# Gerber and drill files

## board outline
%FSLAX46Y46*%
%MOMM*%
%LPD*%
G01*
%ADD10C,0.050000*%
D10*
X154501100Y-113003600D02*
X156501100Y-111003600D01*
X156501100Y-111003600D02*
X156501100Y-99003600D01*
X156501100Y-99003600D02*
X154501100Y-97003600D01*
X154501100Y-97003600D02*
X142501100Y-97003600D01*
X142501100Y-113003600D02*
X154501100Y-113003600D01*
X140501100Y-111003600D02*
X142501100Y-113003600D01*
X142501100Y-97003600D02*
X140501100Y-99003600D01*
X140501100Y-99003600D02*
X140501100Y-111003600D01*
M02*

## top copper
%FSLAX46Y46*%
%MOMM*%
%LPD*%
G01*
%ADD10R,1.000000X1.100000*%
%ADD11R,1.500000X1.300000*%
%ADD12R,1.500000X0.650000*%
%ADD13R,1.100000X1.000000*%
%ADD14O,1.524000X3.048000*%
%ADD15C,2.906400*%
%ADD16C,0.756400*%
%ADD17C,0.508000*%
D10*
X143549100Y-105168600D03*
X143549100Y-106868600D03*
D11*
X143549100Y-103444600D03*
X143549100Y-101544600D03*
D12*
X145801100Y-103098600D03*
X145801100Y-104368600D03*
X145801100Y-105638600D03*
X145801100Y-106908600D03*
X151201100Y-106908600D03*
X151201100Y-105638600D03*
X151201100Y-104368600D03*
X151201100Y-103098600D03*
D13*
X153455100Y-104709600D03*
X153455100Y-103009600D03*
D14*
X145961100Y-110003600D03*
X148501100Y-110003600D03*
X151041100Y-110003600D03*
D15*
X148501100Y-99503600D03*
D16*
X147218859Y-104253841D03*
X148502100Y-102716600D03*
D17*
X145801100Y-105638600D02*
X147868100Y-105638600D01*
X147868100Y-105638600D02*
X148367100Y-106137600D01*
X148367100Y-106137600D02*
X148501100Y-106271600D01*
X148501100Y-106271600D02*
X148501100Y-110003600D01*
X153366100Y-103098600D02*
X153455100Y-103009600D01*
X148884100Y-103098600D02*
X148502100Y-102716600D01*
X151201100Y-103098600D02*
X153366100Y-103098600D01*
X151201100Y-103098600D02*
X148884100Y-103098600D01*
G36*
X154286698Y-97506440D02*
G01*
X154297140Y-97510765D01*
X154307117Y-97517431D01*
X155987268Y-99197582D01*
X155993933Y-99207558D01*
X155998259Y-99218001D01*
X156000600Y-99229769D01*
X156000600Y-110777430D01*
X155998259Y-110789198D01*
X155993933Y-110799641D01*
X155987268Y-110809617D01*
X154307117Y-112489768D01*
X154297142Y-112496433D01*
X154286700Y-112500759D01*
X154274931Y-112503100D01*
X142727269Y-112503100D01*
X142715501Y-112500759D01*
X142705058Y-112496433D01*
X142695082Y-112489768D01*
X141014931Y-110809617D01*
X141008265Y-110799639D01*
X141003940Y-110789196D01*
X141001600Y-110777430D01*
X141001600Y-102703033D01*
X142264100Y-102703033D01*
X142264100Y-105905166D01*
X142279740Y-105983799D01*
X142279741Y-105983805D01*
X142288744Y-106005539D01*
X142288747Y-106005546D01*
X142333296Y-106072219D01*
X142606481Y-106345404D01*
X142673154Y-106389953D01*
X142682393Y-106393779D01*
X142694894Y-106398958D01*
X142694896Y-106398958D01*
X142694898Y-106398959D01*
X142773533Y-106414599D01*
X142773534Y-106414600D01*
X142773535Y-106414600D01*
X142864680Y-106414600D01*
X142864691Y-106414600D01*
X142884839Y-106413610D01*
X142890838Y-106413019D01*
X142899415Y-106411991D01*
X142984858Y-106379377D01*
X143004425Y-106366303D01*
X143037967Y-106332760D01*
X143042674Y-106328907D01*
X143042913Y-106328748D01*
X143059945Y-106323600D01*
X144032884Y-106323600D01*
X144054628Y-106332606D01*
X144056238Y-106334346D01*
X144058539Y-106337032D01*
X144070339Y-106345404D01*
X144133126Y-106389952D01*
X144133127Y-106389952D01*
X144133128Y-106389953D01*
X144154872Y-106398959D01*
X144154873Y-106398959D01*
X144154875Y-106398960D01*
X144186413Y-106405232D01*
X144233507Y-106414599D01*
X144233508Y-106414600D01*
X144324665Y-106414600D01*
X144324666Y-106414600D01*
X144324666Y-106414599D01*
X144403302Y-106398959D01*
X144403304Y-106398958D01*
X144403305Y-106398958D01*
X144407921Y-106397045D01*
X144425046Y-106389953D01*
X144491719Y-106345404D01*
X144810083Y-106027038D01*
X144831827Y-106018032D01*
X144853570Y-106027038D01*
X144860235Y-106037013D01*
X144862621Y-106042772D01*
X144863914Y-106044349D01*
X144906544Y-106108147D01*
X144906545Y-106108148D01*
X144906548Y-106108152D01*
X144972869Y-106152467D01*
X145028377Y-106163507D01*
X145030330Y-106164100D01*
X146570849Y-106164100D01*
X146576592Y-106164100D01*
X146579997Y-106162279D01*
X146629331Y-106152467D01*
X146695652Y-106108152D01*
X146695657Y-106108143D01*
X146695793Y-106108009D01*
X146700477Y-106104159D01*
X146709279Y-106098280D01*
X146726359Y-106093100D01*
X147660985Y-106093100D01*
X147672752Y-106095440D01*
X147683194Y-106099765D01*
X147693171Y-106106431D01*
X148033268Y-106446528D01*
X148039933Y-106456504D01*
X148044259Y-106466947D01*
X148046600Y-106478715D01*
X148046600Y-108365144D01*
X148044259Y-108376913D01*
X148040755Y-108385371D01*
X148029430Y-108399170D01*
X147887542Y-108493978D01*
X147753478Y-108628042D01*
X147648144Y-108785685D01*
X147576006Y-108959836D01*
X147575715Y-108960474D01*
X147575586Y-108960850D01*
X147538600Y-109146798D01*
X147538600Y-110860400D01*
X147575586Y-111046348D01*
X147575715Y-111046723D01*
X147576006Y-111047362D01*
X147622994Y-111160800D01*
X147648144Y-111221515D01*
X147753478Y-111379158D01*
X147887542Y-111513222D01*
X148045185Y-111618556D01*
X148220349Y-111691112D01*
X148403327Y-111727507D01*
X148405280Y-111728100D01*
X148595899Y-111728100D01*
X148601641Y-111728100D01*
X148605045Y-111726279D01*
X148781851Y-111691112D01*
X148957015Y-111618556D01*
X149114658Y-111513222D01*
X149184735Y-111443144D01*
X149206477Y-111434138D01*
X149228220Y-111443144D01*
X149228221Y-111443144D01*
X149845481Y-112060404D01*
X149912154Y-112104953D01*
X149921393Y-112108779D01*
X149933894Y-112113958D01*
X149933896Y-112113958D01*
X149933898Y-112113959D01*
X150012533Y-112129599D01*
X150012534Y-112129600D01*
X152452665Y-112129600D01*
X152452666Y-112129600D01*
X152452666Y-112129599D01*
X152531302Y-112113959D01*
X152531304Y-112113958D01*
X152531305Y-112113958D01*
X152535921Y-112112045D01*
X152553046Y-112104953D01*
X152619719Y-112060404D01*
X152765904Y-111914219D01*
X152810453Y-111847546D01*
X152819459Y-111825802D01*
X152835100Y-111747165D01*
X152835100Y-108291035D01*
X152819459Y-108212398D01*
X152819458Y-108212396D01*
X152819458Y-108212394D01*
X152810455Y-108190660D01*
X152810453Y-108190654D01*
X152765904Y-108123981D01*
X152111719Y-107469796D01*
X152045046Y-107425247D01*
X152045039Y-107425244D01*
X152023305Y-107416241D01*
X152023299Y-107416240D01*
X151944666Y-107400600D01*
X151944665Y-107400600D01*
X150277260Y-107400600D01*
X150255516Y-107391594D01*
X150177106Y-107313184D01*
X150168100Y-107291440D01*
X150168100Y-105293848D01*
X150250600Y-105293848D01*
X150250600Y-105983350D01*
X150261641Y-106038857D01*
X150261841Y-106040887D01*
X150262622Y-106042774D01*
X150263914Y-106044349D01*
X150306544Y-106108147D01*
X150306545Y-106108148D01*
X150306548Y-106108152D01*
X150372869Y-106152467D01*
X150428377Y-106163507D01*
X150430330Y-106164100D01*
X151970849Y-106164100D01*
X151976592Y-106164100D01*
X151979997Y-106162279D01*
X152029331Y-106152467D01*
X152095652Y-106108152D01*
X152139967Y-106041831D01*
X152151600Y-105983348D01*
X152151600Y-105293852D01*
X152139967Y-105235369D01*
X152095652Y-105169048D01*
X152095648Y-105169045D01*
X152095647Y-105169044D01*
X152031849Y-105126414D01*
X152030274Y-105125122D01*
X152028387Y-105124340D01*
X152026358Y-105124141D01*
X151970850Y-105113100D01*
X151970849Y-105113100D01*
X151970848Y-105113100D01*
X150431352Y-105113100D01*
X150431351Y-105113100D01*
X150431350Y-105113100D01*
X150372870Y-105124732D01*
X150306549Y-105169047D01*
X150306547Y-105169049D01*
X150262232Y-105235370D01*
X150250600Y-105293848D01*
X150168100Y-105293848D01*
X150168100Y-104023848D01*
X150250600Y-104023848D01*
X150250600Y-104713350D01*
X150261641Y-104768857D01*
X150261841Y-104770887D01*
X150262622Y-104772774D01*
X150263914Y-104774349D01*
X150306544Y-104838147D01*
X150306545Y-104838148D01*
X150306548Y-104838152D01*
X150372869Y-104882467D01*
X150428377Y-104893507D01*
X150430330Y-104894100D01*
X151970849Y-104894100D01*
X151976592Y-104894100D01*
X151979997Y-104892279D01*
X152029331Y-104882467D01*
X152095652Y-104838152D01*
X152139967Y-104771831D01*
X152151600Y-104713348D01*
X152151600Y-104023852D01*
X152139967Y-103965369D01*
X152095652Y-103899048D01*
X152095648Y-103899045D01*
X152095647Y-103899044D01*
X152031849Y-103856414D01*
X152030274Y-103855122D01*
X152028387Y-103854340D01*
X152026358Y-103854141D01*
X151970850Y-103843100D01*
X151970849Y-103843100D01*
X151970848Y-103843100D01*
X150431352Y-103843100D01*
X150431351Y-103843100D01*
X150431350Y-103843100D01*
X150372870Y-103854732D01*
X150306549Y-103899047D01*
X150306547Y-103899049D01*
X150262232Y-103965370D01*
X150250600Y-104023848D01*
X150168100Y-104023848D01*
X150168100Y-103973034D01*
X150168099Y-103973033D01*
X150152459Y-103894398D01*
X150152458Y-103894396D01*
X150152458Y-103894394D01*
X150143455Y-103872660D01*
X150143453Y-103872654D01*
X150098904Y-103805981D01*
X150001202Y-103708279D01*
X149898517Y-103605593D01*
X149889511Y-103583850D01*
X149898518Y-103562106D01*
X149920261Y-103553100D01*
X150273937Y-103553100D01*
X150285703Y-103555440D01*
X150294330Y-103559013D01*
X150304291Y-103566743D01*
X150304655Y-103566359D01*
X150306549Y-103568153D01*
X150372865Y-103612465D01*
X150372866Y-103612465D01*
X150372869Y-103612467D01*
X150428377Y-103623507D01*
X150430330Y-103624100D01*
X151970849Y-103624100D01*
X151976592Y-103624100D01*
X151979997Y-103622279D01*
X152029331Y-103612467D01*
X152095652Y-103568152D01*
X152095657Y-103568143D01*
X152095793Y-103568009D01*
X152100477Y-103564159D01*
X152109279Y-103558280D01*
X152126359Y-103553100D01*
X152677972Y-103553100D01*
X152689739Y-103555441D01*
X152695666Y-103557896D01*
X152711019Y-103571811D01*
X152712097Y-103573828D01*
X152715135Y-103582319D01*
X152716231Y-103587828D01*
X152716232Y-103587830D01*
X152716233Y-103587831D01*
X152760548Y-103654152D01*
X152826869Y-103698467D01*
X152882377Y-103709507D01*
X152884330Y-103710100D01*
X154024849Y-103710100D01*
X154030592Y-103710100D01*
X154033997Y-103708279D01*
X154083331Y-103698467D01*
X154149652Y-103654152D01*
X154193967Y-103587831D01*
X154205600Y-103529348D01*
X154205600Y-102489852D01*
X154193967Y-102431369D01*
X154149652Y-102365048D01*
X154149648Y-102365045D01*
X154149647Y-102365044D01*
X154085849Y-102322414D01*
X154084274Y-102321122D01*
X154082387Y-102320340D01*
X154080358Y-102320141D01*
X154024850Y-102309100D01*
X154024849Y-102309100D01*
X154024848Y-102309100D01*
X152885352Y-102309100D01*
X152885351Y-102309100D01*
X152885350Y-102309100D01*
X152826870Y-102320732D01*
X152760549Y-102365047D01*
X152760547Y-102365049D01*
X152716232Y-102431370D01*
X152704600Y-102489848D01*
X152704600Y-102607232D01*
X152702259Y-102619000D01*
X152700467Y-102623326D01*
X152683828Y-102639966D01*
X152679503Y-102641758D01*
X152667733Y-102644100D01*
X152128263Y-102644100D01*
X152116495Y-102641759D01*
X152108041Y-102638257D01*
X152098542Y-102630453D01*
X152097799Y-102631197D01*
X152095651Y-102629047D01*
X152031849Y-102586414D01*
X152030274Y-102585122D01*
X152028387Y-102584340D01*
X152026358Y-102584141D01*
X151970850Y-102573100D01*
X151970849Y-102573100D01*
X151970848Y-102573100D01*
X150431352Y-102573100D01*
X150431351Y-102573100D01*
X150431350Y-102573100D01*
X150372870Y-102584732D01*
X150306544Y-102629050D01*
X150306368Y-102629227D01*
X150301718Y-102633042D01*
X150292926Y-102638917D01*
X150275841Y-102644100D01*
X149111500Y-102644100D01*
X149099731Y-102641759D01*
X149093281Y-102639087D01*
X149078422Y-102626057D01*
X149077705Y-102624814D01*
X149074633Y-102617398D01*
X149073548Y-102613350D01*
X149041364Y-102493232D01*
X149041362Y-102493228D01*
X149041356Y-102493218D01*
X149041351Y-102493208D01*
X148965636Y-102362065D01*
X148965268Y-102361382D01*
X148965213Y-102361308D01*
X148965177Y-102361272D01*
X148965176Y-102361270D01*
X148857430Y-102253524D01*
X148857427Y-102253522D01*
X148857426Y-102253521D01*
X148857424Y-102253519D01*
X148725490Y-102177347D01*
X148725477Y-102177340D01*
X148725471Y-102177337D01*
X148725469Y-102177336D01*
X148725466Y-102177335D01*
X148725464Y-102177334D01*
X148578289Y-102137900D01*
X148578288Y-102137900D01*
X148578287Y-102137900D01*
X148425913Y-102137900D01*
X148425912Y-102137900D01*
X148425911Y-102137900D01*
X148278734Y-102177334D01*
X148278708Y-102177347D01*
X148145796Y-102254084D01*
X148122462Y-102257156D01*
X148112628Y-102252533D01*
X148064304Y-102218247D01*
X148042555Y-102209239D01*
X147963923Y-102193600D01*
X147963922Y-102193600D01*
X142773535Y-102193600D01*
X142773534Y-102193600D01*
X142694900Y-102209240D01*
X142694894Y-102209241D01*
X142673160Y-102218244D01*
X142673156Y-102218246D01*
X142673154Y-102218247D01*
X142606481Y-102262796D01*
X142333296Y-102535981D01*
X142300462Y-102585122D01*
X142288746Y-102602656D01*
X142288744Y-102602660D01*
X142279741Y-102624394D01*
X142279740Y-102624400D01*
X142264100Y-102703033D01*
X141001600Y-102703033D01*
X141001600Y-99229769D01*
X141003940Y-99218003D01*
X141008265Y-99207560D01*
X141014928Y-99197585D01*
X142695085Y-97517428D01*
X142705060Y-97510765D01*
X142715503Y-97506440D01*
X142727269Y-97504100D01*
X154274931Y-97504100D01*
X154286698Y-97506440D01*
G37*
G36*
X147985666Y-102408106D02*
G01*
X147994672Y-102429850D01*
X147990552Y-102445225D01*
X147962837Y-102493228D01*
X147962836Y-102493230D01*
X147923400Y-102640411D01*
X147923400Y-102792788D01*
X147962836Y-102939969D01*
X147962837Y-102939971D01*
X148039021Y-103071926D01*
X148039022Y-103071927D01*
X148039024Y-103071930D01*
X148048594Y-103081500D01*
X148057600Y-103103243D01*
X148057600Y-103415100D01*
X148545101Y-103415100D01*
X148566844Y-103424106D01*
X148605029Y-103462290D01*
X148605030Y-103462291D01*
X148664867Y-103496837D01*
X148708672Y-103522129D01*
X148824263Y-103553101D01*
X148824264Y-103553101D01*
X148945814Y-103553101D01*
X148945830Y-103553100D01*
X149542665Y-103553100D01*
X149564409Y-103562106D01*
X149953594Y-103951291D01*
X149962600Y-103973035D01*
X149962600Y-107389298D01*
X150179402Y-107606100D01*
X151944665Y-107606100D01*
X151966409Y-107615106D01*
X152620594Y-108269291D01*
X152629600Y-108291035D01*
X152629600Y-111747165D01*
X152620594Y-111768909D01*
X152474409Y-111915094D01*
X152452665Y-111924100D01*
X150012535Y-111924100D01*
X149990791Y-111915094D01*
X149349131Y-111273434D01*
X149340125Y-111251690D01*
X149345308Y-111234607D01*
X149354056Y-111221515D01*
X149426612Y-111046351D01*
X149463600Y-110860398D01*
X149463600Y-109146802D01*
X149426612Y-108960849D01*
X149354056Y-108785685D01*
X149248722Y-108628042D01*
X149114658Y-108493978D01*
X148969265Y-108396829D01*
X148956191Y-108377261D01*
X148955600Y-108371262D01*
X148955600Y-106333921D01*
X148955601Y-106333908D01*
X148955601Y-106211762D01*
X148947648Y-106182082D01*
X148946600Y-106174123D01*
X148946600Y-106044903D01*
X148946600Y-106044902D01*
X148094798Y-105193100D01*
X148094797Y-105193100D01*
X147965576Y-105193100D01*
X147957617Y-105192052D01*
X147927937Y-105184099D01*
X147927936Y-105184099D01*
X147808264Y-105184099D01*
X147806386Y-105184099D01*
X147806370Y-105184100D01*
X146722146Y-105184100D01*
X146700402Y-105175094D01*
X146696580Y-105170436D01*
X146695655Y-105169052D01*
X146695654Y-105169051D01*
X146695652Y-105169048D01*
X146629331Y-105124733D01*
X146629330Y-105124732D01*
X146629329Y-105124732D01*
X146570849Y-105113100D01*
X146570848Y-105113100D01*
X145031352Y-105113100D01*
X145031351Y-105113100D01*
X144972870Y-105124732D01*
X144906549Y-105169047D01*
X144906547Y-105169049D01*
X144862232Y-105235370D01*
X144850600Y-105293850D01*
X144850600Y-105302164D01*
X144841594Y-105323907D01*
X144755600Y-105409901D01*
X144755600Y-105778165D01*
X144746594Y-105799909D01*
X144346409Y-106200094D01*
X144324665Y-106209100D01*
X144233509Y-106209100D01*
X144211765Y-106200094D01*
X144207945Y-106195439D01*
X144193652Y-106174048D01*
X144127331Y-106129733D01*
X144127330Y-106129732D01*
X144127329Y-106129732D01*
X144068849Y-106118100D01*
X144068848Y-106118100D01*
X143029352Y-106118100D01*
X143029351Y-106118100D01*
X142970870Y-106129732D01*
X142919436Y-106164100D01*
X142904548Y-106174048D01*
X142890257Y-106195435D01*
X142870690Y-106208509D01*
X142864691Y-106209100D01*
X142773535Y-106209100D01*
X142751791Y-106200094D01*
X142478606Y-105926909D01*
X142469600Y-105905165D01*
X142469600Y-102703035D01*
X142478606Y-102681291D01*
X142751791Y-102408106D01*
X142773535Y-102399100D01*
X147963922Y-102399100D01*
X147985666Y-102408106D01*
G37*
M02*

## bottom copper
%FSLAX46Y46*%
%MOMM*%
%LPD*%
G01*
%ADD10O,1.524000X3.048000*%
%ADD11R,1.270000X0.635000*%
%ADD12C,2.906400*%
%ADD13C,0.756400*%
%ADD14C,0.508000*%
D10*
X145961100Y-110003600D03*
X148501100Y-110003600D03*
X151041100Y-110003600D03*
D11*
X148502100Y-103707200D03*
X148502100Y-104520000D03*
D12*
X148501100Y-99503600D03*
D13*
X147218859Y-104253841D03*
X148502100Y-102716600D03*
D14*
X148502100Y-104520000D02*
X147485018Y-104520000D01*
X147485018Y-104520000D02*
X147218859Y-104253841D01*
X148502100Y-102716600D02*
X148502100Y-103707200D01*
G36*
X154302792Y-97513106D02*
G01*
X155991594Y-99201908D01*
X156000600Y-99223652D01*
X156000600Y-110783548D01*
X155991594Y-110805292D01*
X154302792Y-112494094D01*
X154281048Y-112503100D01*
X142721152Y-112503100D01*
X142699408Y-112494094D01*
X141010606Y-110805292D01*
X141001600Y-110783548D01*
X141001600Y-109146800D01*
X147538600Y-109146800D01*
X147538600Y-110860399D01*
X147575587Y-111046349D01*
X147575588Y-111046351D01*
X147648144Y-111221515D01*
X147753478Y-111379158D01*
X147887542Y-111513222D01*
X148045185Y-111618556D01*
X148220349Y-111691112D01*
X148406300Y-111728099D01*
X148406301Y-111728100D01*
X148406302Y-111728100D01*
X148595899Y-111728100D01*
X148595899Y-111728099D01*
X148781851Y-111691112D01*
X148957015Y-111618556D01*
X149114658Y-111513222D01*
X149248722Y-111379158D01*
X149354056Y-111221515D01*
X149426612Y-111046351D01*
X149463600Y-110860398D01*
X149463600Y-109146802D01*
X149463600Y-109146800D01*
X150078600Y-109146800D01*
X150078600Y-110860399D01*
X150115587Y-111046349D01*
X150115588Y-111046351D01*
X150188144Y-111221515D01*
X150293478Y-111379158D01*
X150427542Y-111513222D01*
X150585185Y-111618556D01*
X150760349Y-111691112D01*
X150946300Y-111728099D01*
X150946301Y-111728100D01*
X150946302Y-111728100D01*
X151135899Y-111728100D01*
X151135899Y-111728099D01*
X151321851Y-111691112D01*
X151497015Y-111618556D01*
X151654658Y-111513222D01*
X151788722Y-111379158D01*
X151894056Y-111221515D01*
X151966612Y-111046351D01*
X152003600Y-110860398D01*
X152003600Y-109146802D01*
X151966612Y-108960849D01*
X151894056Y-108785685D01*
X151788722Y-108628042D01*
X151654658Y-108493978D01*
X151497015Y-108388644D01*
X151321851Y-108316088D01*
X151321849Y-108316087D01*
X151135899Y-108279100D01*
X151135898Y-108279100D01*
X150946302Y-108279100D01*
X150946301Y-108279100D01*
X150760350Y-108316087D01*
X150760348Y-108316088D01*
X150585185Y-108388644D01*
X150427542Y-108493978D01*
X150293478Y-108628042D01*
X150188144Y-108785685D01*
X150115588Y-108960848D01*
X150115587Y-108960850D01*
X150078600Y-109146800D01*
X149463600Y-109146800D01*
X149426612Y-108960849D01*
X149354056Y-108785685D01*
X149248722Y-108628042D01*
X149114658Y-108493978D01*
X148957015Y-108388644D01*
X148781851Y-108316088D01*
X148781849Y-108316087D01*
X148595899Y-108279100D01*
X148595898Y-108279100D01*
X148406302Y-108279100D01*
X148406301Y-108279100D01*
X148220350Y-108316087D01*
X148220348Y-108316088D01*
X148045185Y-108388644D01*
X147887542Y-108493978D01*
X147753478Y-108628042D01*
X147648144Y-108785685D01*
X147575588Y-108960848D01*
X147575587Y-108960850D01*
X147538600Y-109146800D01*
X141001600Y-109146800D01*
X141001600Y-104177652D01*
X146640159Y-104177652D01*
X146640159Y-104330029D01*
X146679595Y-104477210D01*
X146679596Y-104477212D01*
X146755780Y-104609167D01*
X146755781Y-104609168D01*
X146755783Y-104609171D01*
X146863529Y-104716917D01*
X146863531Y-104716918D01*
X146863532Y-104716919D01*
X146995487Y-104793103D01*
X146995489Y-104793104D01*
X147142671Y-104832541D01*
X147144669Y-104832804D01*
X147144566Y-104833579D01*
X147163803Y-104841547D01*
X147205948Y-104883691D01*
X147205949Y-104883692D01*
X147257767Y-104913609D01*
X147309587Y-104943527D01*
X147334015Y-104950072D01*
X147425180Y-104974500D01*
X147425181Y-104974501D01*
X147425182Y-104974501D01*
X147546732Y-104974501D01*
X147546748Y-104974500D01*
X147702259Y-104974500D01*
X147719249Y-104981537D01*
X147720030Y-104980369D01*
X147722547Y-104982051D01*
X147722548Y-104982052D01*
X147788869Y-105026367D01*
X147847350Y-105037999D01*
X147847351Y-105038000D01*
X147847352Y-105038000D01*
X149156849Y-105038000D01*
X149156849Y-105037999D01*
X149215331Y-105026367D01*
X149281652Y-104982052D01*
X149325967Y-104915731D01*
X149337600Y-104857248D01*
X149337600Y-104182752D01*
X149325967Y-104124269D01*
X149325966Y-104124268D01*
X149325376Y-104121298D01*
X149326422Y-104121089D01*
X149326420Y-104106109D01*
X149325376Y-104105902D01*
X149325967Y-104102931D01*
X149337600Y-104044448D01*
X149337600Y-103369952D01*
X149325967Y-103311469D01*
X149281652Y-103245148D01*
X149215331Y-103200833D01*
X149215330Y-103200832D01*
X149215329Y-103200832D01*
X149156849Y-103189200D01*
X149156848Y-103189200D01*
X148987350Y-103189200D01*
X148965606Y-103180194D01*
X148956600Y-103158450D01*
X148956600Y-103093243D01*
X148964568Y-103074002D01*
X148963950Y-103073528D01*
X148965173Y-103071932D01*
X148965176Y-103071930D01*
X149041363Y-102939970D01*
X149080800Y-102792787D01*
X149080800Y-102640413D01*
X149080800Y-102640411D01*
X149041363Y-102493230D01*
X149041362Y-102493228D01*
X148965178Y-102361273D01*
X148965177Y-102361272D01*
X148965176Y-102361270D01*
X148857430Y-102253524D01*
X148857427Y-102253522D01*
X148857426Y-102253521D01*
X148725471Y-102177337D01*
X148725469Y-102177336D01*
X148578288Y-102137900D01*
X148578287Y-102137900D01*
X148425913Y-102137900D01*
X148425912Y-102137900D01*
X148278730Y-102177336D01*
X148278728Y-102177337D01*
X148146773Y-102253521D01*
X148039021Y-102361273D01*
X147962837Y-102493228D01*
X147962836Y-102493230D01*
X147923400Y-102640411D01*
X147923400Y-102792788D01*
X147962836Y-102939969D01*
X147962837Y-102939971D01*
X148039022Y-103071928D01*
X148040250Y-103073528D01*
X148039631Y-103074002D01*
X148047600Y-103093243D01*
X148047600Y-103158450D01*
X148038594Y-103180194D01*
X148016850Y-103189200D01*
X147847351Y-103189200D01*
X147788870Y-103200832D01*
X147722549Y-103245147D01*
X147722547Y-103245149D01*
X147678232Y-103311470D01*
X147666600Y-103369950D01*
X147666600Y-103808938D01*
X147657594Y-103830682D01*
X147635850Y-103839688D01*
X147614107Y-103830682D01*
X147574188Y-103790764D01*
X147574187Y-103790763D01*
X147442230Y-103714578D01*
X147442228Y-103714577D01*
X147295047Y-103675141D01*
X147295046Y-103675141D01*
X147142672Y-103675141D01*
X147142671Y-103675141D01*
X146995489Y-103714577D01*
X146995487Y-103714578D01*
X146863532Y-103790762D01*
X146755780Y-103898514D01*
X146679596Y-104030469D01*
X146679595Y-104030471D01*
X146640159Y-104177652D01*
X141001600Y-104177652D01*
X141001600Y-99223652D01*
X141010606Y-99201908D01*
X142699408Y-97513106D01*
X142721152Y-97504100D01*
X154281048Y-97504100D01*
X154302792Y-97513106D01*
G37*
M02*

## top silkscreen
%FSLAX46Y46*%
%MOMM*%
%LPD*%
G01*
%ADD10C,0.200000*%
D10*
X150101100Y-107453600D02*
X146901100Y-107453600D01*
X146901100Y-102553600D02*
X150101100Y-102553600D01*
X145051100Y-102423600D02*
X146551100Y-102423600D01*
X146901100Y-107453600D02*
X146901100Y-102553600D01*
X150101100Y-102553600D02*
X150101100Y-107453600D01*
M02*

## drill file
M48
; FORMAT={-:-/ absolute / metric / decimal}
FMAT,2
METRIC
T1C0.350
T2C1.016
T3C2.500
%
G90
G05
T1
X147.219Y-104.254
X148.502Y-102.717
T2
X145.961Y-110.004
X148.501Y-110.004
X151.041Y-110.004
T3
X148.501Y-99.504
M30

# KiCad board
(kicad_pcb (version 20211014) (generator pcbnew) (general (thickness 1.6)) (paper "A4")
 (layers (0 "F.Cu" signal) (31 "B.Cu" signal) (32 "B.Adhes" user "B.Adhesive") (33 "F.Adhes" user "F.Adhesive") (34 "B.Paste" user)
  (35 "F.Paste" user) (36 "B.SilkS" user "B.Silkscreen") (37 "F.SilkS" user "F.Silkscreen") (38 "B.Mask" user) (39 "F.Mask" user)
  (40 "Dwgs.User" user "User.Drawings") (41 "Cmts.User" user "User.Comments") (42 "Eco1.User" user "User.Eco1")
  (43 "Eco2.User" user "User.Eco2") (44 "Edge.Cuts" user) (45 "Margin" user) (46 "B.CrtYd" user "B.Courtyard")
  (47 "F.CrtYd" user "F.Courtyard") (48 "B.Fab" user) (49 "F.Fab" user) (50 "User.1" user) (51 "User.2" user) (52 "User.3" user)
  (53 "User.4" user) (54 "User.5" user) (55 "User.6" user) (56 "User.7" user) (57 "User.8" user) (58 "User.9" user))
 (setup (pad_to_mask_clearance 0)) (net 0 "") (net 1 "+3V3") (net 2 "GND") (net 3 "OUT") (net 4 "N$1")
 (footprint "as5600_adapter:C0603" (layer "F.Cu") (at 143.5491 106.0186 -90)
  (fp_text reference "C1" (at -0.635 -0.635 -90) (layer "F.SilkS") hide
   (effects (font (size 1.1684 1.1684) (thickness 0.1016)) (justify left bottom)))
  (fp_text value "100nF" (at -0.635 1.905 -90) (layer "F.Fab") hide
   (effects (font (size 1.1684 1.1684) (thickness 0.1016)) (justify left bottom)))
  (pad "1" smd rect (at -0.85 0 270) (size 1.1 1) (layers "F.Cu" "F.Paste" "F.Mask") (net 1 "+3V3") (solder_mask_margin 0.1016))
  (pad "2" smd rect (at 0.85 0 270) (size 1.1 1) (layers "F.Cu" "F.Paste" "F.Mask") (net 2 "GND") (solder_mask_margin 0.1016)))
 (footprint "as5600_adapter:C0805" (layer "F.Cu") (at 143.5491 102.4946 90)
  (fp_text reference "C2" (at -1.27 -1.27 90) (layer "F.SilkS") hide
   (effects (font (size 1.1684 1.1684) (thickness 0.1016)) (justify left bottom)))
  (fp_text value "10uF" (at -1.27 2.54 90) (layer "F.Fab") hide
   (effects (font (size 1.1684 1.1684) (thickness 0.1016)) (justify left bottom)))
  (pad "1" smd rect (at -0.95 0 90) (size 1.3 1.5) (layers "F.Cu" "F.Paste" "F.Mask") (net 1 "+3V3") (solder_mask_margin 0.1016))
  (pad "2" smd rect (at 0.95 0 90) (size 1.3 1.5) (layers "F.Cu" "F.Paste" "F.Mask") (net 2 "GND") (solder_mask_margin 0.1016)))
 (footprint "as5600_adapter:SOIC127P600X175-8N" (layer "F.Cu") (at 148.5011 105.0036)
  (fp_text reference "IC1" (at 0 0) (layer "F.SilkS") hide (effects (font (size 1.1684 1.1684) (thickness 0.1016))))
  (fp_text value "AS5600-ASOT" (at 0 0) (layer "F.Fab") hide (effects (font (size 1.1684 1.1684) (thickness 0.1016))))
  (fp_line (start 1.6 2.45) (end -1.6 2.45) (layer "F.SilkS") (width 0.2))
  (fp_line (start -1.6 -2.45) (end 1.6 -2.45) (layer "F.SilkS") (width 0.2))
  (fp_line (start -3.45 -2.58) (end -1.95 -2.58) (layer "F.SilkS") (width 0.2))
  (fp_line (start -1.6 2.45) (end -1.6 -2.45) (layer "F.SilkS") (width 0.2))
  (fp_line (start 1.6 -2.45) (end 1.6 2.45) (layer "F.SilkS") (width 0.2))
  (pad "1" smd rect (at -2.7 -1.905) (size 1.5 0.65) (layers "F.Cu" "F.Paste" "F.Mask") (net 1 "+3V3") (solder_mask_margin 0.1016))
  (pad "2" smd rect (at -2.7 -0.635) (size 1.5 0.65) (layers "F.Cu" "F.Paste" "F.Mask") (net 1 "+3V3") (solder_mask_margin 0.1016))
  (pad "3" smd rect (at -2.7 0.635) (size 1.5 0.65) (layers "F.Cu" "F.Paste" "F.Mask") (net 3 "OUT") (solder_mask_margin 0.1016))
  (pad "4" smd rect (at -2.7 1.905) (size 1.5 0.65) (layers "F.Cu" "F.Paste" "F.Mask") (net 2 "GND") (solder_mask_margin 0.1016))
  (pad "5" smd rect (at 2.7 1.905) (size 1.5 0.65) (layers "F.Cu" "F.Paste" "F.Mask") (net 2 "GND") (solder_mask_margin 0.1016))
  (pad "6" smd rect (at 2.7 0.635) (size 1.5 0.65) (layers "F.Cu" "F.Paste" "F.Mask") (solder_mask_margin 0.1016))
  (pad "7" smd rect (at 2.7 -0.635) (size 1.5 0.65) (layers "F.Cu" "F.Paste" "F.Mask") (solder_mask_margin 0.1016))
  (pad "8" smd rect (at 2.7 -1.905) (size 1.5 0.65) (layers "F.Cu" "F.Paste" "F.Mask") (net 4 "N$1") (solder_mask_margin 0.1016)))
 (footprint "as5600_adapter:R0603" (layer "F.Cu") (at 153.4551 103.8596 90)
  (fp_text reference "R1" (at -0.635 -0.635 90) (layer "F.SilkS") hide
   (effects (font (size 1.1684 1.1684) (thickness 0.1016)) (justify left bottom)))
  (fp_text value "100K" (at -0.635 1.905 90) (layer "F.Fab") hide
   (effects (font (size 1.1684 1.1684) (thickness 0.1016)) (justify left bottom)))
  (pad "1" smd rect (at -0.85 0 90) (size 1 1.1) (layers "F.Cu" "F.Paste" "F.Mask") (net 2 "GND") (solder_mask_margin 0.1016))
  (pad "2" smd rect (at 0.85 0 90) (size 1 1.1) (layers "F.Cu" "F.Paste" "F.Mask") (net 4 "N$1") (solder_mask_margin 0.1016)))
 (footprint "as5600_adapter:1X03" (layer "B.Cu") (at 148.5011 110.0036)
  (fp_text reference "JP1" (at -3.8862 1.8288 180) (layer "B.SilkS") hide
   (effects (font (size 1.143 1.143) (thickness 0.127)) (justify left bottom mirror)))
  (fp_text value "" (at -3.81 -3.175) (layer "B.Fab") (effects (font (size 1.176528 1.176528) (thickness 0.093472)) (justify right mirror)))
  (pad "1" thru_hole oval (at -2.54 0 270) (size 3.048 1.524) (drill 1.016) (layers *.Cu *.Mask) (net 2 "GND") (solder_mask_margin 0.1016))
  (pad "2" thru_hole oval (at 0 0 270) (size 3.048 1.524) (drill 1.016) (layers *.Cu *.Mask) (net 3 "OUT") (solder_mask_margin 0.1016))
  (pad "3" thru_hole oval (at 2.54 0 270) (size 3.048 1.524) (drill 1.016) (layers *.Cu *.Mask) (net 1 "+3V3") (solder_mask_margin 0.1016)))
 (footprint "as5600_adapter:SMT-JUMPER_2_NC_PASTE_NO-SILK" (layer "B.Cu") (at 148.5021 104.1136 -90)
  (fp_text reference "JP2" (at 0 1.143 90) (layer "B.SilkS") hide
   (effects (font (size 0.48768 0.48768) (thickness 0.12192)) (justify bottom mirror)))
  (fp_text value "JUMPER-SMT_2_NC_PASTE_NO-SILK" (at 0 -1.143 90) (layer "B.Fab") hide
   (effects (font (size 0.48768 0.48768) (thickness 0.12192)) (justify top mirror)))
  (pad "1" smd rect (at -0.4064 0 270) (size 0.635 1.27) (layers "B.Cu" "B.Mask") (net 4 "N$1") (solder_mask_margin 0.1016))
  (pad "2" smd rect (at 0.4064 0 270) (size 0.635 1.27) (layers "B.Cu" "B.Mask") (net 1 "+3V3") (solder_mask_margin 0.1016)))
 (gr_line (start 154.5011 113.0036) (end 156.5011 111.0036) (layer "Edge.Cuts") (width 0.05))
 (gr_line (start 156.5011 111.0036) (end 156.5011 99.0036) (layer "Edge.Cuts") (width 0.05))
 (gr_line (start 156.5011 99.0036) (end 154.5011 97.0036) (layer "Edge.Cuts") (width 0.05))
 (gr_line (start 154.5011 97.0036) (end 142.5011 97.0036) (layer "Edge.Cuts") (width 0.05))
 (gr_line (start 142.5011 113.0036) (end 154.5011 113.0036) (layer "Edge.Cuts") (width 0.05))
 (gr_line (start 140.5011 111.0036) (end 142.5011 113.0036) (layer "Edge.Cuts") (width 0.05))
 (gr_line (start 142.5011 97.0036) (end 140.5011 99.0036) (layer "Edge.Cuts") (width 0.05))
 (gr_line (start 140.5011 99.0036) (end 140.5011 111.0036) (layer "Edge.Cuts") (width 0.05))
 (via (at 148.5011 99.5036) (size 2.9064) (drill 2.5) (layers "F.Cu" "B.Cu") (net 2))
 (segment (start 145.8011 105.6386) (end 147.8681 105.6386) (width 0.508) (layer "F.Cu") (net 3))
 (segment (start 147.8681 105.6386) (end 148.3671 106.1376) (width 0.508) (layer "F.Cu") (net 3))
 (segment (start 148.3671 106.1376) (end 148.5011 106.2716) (width 0.508) (layer "F.Cu") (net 3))
 (segment (start 148.5011 106.2716) (end 148.5011 110.0036) (width 0.508) (layer "F.Cu") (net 3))
 (via (at 147.218859 104.253841) (size 0.7564) (drill 0.35) (layers "F.Cu" "B.Cu") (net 1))
 (segment (start 148.5021 104.52) (end 147.485018 104.52) (width 0.508) (layer "B.Cu") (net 1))
 (segment (start 147.485018 104.52) (end 147.218859 104.253841) (width 0.508) (layer "B.Cu") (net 1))
 (segment (start 153.3661 103.0986) (end 153.4551 103.0096) (width 0.508) (layer "F.Cu") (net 4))
 (segment (start 148.8841 103.0986) (end 148.5021 102.7166) (width 0.508) (layer "F.Cu") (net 4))
 (segment (start 151.2011 103.0986) (end 153.3661 103.0986) (width 0.508) (layer "F.Cu") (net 4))
 (segment (start 151.2011 103.0986) (end 148.8841 103.0986) (width 0.508) (layer "F.Cu") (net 4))
 (via (at 148.5021 102.7166) (size 0.7564) (drill 0.35) (layers "F.Cu" "B.Cu") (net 4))
 (segment (start 148.5021 102.7166) (end 148.5021 103.7072) (width 0.508) (layer "B.Cu") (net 4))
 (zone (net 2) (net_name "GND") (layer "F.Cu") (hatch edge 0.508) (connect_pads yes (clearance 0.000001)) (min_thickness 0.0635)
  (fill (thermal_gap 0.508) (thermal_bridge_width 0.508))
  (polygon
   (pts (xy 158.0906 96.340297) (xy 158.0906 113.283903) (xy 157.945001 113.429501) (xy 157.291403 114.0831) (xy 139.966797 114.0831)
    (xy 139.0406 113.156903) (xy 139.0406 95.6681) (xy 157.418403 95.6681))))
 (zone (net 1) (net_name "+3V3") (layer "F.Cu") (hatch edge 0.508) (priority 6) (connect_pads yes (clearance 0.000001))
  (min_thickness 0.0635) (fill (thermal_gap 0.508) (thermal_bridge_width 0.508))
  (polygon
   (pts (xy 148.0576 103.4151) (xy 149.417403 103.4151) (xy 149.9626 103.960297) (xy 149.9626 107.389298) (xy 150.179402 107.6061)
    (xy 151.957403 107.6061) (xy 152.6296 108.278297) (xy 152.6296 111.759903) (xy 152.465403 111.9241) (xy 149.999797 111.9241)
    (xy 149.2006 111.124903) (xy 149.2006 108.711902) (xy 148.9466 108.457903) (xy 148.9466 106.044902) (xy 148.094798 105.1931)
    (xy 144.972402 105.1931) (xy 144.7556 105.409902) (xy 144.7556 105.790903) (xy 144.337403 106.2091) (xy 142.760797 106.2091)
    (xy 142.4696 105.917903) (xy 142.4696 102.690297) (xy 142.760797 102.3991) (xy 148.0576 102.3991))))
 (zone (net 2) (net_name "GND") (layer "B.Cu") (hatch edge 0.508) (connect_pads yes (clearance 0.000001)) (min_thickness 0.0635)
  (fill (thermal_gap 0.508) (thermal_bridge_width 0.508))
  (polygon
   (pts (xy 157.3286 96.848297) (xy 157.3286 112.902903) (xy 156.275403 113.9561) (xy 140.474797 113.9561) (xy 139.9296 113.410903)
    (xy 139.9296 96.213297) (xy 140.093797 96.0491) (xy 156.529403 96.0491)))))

